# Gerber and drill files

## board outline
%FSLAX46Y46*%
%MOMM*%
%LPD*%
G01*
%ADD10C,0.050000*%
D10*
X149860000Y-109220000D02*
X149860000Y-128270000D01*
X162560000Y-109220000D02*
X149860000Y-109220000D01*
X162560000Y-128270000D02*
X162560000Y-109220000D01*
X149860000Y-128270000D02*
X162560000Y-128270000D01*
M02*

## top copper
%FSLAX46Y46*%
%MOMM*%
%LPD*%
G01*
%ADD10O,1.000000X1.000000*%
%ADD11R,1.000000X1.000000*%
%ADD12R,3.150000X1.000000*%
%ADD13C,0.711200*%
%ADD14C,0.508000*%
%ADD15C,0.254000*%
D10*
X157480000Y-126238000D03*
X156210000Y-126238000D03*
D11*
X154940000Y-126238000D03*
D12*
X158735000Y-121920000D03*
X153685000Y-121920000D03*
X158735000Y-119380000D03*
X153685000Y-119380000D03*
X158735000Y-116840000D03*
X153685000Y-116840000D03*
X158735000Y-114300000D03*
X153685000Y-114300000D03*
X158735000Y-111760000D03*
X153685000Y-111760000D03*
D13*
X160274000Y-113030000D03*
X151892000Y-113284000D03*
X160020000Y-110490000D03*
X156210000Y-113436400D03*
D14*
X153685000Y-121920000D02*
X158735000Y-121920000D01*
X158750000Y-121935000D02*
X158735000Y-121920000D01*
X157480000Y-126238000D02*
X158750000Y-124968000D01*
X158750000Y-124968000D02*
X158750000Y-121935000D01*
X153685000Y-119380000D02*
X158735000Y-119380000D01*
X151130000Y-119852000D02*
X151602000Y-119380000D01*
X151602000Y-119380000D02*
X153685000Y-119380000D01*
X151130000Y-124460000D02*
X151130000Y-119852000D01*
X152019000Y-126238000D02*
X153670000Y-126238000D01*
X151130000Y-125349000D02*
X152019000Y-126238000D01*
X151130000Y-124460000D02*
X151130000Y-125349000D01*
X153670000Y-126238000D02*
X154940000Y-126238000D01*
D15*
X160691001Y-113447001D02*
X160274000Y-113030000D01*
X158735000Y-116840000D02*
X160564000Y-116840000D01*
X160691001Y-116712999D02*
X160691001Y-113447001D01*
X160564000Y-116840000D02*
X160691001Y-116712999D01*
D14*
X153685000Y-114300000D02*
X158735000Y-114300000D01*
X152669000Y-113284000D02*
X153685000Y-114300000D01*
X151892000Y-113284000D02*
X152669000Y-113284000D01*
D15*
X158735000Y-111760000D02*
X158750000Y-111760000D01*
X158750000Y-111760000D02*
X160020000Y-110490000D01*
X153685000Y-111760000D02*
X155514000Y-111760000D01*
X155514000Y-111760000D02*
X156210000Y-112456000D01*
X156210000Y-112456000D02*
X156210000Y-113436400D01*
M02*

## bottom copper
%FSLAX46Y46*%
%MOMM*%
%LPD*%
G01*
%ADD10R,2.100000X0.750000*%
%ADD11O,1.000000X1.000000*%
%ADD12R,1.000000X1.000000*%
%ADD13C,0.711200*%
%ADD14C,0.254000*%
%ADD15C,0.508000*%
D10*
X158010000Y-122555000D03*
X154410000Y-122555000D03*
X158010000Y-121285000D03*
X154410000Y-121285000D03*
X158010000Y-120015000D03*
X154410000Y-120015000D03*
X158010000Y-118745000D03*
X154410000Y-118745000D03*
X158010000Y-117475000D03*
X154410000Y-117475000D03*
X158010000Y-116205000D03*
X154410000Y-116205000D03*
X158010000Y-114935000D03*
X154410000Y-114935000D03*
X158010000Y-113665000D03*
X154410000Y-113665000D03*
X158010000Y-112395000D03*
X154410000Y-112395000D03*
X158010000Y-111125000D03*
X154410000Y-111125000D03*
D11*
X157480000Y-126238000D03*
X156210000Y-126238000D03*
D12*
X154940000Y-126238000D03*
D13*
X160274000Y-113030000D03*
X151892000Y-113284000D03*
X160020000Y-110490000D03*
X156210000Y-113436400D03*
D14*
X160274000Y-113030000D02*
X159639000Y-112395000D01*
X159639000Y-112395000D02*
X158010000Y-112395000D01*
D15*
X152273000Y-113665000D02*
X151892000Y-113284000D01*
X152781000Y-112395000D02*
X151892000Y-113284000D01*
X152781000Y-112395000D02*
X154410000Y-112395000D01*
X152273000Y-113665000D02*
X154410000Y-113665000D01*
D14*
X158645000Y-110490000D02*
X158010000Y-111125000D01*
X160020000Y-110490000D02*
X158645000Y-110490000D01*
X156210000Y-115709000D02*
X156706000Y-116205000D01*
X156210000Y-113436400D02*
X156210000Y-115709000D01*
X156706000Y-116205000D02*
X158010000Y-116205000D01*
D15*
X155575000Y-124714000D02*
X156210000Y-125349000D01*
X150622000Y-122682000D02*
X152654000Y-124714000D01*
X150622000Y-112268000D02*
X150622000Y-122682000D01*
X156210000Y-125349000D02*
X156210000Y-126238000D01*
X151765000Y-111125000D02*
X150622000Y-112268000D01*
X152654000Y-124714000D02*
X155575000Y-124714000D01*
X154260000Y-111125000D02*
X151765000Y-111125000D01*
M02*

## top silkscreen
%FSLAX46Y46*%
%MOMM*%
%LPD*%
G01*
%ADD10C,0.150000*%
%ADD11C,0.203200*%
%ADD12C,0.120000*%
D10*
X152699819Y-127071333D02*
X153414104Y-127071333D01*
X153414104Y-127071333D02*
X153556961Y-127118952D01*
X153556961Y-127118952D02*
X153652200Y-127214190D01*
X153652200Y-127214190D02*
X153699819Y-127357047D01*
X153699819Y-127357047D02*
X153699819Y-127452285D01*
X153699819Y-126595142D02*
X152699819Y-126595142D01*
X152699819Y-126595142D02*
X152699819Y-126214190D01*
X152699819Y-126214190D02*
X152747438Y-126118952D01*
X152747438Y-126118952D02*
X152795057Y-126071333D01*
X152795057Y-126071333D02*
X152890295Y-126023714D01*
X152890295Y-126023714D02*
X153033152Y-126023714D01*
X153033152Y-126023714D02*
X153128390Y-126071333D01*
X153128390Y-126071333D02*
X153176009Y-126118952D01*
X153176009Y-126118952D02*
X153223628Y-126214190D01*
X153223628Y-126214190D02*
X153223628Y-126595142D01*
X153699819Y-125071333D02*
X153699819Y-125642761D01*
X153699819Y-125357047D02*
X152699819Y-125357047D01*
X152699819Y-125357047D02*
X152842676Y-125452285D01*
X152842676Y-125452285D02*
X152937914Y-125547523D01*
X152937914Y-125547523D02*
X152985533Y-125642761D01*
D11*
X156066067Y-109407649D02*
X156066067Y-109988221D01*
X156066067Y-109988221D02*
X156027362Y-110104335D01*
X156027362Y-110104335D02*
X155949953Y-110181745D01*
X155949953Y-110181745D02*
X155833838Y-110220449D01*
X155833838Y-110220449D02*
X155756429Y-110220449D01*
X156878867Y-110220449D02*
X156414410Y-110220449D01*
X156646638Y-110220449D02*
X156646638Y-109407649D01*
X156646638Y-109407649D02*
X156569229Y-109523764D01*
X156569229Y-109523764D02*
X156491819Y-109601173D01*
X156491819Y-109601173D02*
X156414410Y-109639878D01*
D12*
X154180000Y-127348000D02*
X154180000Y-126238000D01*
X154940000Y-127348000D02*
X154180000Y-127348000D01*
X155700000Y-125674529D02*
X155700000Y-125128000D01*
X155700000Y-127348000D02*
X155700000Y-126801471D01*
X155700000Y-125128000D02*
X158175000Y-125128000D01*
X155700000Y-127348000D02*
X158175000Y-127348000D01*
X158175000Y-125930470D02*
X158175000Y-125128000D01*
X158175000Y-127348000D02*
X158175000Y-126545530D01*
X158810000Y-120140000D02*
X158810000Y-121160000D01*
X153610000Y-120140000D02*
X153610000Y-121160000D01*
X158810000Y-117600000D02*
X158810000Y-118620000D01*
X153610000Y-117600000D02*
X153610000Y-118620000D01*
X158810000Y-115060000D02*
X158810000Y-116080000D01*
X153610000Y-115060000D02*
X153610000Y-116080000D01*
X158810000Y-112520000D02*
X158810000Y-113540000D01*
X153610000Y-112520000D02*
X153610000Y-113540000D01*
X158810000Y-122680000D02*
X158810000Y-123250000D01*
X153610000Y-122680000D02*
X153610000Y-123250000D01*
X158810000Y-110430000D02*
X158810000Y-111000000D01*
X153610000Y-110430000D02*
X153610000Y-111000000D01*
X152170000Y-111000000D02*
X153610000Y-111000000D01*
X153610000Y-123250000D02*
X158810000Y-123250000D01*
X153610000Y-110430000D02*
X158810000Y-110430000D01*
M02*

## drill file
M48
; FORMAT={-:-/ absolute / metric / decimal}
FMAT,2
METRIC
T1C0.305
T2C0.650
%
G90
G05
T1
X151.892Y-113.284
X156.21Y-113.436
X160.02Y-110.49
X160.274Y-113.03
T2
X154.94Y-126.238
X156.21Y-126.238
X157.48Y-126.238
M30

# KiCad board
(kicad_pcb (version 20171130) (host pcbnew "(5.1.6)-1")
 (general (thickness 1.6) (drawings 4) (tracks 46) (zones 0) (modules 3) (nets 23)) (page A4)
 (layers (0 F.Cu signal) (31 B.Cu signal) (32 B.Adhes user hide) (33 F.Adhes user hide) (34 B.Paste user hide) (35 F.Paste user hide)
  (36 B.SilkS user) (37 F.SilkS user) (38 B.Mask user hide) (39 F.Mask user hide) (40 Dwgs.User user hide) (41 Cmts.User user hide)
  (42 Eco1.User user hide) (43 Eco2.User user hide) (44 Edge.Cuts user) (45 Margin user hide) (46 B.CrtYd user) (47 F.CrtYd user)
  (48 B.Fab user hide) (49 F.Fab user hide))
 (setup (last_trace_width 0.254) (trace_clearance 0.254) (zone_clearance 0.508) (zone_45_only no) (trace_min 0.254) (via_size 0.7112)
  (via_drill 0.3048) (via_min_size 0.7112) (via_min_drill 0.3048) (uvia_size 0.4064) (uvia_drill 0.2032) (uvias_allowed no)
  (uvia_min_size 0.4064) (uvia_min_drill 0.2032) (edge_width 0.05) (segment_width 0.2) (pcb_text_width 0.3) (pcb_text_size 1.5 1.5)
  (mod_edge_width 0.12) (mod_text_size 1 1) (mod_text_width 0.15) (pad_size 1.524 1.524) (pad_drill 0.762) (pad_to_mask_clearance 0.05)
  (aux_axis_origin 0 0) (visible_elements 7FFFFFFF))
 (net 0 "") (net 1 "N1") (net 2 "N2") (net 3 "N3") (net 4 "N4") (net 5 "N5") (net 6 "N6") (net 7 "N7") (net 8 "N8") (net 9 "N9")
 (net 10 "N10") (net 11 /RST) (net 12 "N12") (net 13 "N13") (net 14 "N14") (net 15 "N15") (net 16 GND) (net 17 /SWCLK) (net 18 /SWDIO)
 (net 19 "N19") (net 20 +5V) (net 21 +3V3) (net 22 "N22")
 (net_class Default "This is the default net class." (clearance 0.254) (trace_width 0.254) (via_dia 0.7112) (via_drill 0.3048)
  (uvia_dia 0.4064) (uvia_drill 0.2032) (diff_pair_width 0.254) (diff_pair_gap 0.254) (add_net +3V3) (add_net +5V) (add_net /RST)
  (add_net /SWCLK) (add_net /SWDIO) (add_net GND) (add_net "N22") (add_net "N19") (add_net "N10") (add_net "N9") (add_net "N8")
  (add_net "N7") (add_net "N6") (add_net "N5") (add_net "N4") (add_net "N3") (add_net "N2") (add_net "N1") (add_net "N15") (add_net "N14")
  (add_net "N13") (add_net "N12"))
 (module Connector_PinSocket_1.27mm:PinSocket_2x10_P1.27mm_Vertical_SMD (layer B.Cu) (at 156.21 116.84 180)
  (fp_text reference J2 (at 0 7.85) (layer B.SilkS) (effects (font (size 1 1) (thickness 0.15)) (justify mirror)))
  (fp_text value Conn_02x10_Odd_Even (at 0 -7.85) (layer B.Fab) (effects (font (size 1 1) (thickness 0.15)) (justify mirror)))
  (pad 20 smd rect (at -1.8 -5.715 180) (size 2.1 0.75) (layers B.Cu B.Paste B.Mask) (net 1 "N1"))
  (pad 19 smd rect (at 1.8 -5.715 180) (size 2.1 0.75) (layers B.Cu B.Paste B.Mask) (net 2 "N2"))
  (pad 18 smd rect (at -1.8 -4.445 180) (size 2.1 0.75) (layers B.Cu B.Paste B.Mask) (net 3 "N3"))
  (pad 17 smd rect (at 1.8 -4.445 180) (size 2.1 0.75) (layers B.Cu B.Paste B.Mask) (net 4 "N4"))
  (pad 16 smd rect (at -1.8 -3.175 180) (size 2.1 0.75) (layers B.Cu B.Paste B.Mask) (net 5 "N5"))
  (pad 15 smd rect (at 1.8 -3.175 180) (size 2.1 0.75) (layers B.Cu B.Paste B.Mask) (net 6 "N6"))
  (pad 14 smd rect (at -1.8 -1.905 180) (size 2.1 0.75) (layers B.Cu B.Paste B.Mask) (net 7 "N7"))
  (pad 13 smd rect (at 1.8 -1.905 180) (size 2.1 0.75) (layers B.Cu B.Paste B.Mask) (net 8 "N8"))
  (pad 12 smd rect (at -1.8 -0.635 180) (size 2.1 0.75) (layers B.Cu B.Paste B.Mask) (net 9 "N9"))
  (pad 11 smd rect (at 1.8 -0.635 180) (size 2.1 0.75) (layers B.Cu B.Paste B.Mask) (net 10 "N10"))
  (pad 10 smd rect (at -1.8 0.635 180) (size 2.1 0.75) (layers B.Cu B.Paste B.Mask) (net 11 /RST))
  (pad 9 smd rect (at 1.8 0.635 180) (size 2.1 0.75) (layers B.Cu B.Paste B.Mask) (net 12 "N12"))
  (pad 8 smd rect (at -1.8 1.905 180) (size 2.1 0.75) (layers B.Cu B.Paste B.Mask) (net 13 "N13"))
  (pad 7 smd rect (at 1.8 1.905 180) (size 2.1 0.75) (layers B.Cu B.Paste B.Mask) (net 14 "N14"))
  (pad 6 smd rect (at -1.8 3.175 180) (size 2.1 0.75) (layers B.Cu B.Paste B.Mask) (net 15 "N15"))
  (pad 5 smd rect (at 1.8 3.175 180) (size 2.1 0.75) (layers B.Cu B.Paste B.Mask) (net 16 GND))
  (pad 4 smd rect (at -1.8 4.445 180) (size 2.1 0.75) (layers B.Cu B.Paste B.Mask) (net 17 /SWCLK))
  (pad 3 smd rect (at 1.8 4.445 180) (size 2.1 0.75) (layers B.Cu B.Paste B.Mask) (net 16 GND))
  (pad 2 smd rect (at -1.8 5.715 180) (size 2.1 0.75) (layers B.Cu B.Paste B.Mask) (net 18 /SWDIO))
  (pad 1 smd rect (at 1.8 5.715 180) (size 2.1 0.75) (layers B.Cu B.Paste B.Mask) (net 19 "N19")))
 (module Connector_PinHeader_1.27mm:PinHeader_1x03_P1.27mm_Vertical (layer F.Cu) (at 154.94 126.238 90)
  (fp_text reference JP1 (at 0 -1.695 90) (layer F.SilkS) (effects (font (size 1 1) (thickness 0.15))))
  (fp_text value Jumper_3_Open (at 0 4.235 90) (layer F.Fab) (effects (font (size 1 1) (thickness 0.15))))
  (fp_line (start -1.11 -0.76) (end 0 -0.76) (layer F.SilkS) (width 0.12))
  (fp_line (start -1.11 0) (end -1.11 -0.76) (layer F.SilkS) (width 0.12))
  (fp_line (start 0.563471 0.76) (end 1.11 0.76) (layer F.SilkS) (width 0.12))
  (fp_line (start -1.11 0.76) (end -0.563471 0.76) (layer F.SilkS) (width 0.12))
  (fp_line (start 1.11 0.76) (end 1.11 3.235) (layer F.SilkS) (width 0.12))
  (fp_line (start -1.11 0.76) (end -1.11 3.235) (layer F.SilkS) (width 0.12))
  (fp_line (start 0.30753 3.235) (end 1.11 3.235) (layer F.SilkS) (width 0.12))
  (fp_line (start -1.11 3.235) (end -0.30753 3.235) (layer F.SilkS) (width 0.12))
  (pad 3 thru_hole oval (at 0 2.54 90) (size 1 1) (drill 0.65) (layers *.Cu *.Mask) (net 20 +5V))
  (pad 2 thru_hole oval (at 0 1.27 90) (size 1 1) (drill 0.65) (layers *.Cu *.Mask) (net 19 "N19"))
  (pad 1 thru_hole rect (at 0 0 90) (size 1 1) (drill 0.65) (layers *.Cu *.Mask) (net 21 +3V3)))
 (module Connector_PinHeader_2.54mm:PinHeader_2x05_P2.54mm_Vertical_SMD (layer F.Cu) (at 156.21 116.84)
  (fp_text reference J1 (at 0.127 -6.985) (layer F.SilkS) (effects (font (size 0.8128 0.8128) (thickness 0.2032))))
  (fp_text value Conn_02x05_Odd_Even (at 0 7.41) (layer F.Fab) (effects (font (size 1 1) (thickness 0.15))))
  (fp_line (start 2.6 3.3) (end 2.6 4.32) (layer F.SilkS) (width 0.12))
  (fp_line (start -2.6 3.3) (end -2.6 4.32) (layer F.SilkS) (width 0.12))
  (fp_line (start 2.6 0.76) (end 2.6 1.78) (layer F.SilkS) (width 0.12))
  (fp_line (start -2.6 0.76) (end -2.6 1.78) (layer F.SilkS) (width 0.12))
  (fp_line (start 2.6 -1.78) (end 2.6 -0.76) (layer F.SilkS) (width 0.12))
  (fp_line (start -2.6 -1.78) (end -2.6 -0.76) (layer F.SilkS) (width 0.12))
  (fp_line (start 2.6 -4.32) (end 2.6 -3.3) (layer F.SilkS) (width 0.12))
  (fp_line (start -2.6 -4.32) (end -2.6 -3.3) (layer F.SilkS) (width 0.12))
  (fp_line (start 2.6 5.84) (end 2.6 6.41) (layer F.SilkS) (width 0.12))
  (fp_line (start -2.6 5.84) (end -2.6 6.41) (layer F.SilkS) (width 0.12))
  (fp_line (start 2.6 -6.41) (end 2.6 -5.84) (layer F.SilkS) (width 0.12))
  (fp_line (start -2.6 -6.41) (end -2.6 -5.84) (layer F.SilkS) (width 0.12))
  (fp_line (start -4.04 -5.84) (end -2.6 -5.84) (layer F.SilkS) (width 0.12))
  (fp_line (start -2.6 6.41) (end 2.6 6.41) (layer F.SilkS) (width 0.12))
  (fp_line (start -2.6 -6.41) (end 2.6 -6.41) (layer F.SilkS) (width 0.12))
  (pad 10 smd rect (at 2.525 5.08) (size 3.15 1) (layers F.Cu F.Paste F.Mask) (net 20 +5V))
  (pad 9 smd rect (at -2.525 5.08) (size 3.15 1) (layers F.Cu F.Paste F.Mask) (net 20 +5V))
  (pad 8 smd rect (at 2.525 2.54) (size 3.15 1) (layers F.Cu F.Paste F.Mask) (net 21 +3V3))
  (pad 7 smd rect (at -2.525 2.54) (size 3.15 1) (layers F.Cu F.Paste F.Mask) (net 21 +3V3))
  (pad 6 smd rect (at 2.525 0) (size 3.15 1) (layers F.Cu F.Paste F.Mask) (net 17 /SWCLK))
  (pad 5 smd rect (at -2.525 0) (size 3.15 1) (layers F.Cu F.Paste F.Mask) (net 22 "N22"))
  (pad 4 smd rect (at 2.525 -2.54) (size 3.15 1) (layers F.Cu F.Paste F.Mask) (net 16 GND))
  (pad 3 smd rect (at -2.525 -2.54) (size 3.15 1) (layers F.Cu F.Paste F.Mask) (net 16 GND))
  (pad 2 smd rect (at 2.525 -5.08) (size 3.15 1) (layers F.Cu F.Paste F.Mask) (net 18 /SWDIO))
  (pad 1 smd rect (at -2.525 -5.08) (size 3.15 1) (layers F.Cu F.Paste F.Mask) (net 11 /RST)))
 (gr_line (start 149.86 109.22) (end 149.86 128.27) (layer Edge.Cuts) (width 0.05))
 (gr_line (start 162.56 109.22) (end 149.86 109.22) (layer Edge.Cuts) (width 0.05))
 (gr_line (start 162.56 128.27) (end 162.56 109.22) (layer Edge.Cuts) (width 0.05))
 (gr_line (start 149.86 128.27) (end 162.56 128.27) (layer Edge.Cuts) (width 0.05))
 (segment (start 153.685 121.92) (end 158.735 121.92) (width 0.508) (layer F.Cu) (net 20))
 (segment (start 158.75 121.935) (end 158.735 121.92) (width 0.508) (layer F.Cu) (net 20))
 (segment (start 157.48 126.238) (end 158.75 124.968) (width 0.508) (layer F.Cu) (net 20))
 (segment (start 158.75 124.968) (end 158.75 121.935) (width 0.508) (layer F.Cu) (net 20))
 (segment (start 153.685 119.38) (end 158.735 119.38) (width 0.508) (layer F.Cu) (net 21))
 (segment (start 151.13 119.852) (end 151.602 119.38) (width 0.508) (layer F.Cu) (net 21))
 (segment (start 151.602 119.38) (end 153.685 119.38) (width 0.508) (layer F.Cu) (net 21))
 (segment (start 151.13 124.46) (end 151.13 119.852) (width 0.508) (layer F.Cu) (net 21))
 (segment (start 152.019 126.238) (end 153.67 126.238) (width 0.508) (layer F.Cu) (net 21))
 (segment (start 151.13 125.349) (end 152.019 126.238) (width 0.508) (layer F.Cu) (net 21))
 (segment (start 151.13 124.46) (end 151.13 125.349) (width 0.508) (layer F.Cu) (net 21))
 (segment (start 153.67 126.238) (end 154.94 126.238) (width 0.508) (layer F.Cu) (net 21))
 (segment (start 160.691001 113.447001) (end 160.274 113.03) (width 0.254) (layer F.Cu) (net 17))
 (via (at 160.274 113.03) (size 0.7112) (drill 0.3048) (layers F.Cu B.Cu) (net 17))
 (segment (start 158.735 116.84) (end 160.564 116.84) (width 0.254) (layer F.Cu) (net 17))
 (segment (start 160.691001 116.712999) (end 160.691001 113.447001) (width 0.254) (layer F.Cu) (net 17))
 (segment (start 160.564 116.84) (end 160.691001 116.712999) (width 0.254) (layer F.Cu) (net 17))
 (segment (start 160.274 113.03) (end 159.639 112.395) (width 0.254) (layer B.Cu) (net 17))
 (segment (start 159.639 112.395) (end 158.01 112.395) (width 0.254) (layer B.Cu) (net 17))
 (segment (start 153.685 114.3) (end 158.735 114.3) (width 0.508) (layer F.Cu) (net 16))
 (via (at 151.892 113.284) (size 0.7112) (drill 0.3048) (layers F.Cu B.Cu) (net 16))
 (segment (start 152.273 113.665) (end 151.892 113.284) (width 0.508) (layer B.Cu) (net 16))
 (segment (start 152.669 113.284) (end 153.685 114.3) (width 0.508) (layer F.Cu) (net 16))
 (segment (start 151.892 113.284) (end 152.669 113.284) (width 0.508) (layer F.Cu) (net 16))
 (segment (start 152.781 112.395) (end 151.892 113.284) (width 0.508) (layer B.Cu) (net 16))
 (segment (start 152.781 112.395) (end 154.41 112.395) (width 0.508) (layer B.Cu) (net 16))
 (segment (start 152.273 113.665) (end 154.41 113.665) (width 0.508) (layer B.Cu) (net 16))
 (via (at 160.02 110.49) (size 0.7112) (drill 0.3048) (layers F.Cu B.Cu) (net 18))
 (segment (start 158.735 111.76) (end 158.75 111.76) (width 0.254) (layer F.Cu) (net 18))
 (segment (start 158.75 111.76) (end 160.02 110.49) (width 0.254) (layer F.Cu) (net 18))
 (segment (start 158.645 110.49) (end 158.01 111.125) (width 0.254) (layer B.Cu) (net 18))
 (segment (start 160.02 110.49) (end 158.645 110.49) (width 0.254) (layer B.Cu) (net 18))
 (segment (start 153.685 111.76) (end 155.514 111.76) (width 0.254) (layer F.Cu) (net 11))
 (segment (start 155.514 111.76) (end 156.21 112.456) (width 0.254) (layer F.Cu) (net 11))
 (via (at 156.21 113.4364) (size 0.7112) (drill 0.3048) (layers F.Cu B.Cu) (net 11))
 (segment (start 156.21 112.456) (end 156.21 113.4364) (width 0.254) (layer F.Cu) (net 11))
 (segment (start 156.21 115.709) (end 156.706 116.205) (width 0.254) (layer B.Cu) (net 11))
 (segment (start 156.21 113.4364) (end 156.21 115.709) (width 0.254) (layer B.Cu) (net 11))
 (segment (start 156.706 116.205) (end 158.01 116.205) (width 0.254) (layer B.Cu) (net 11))
 (segment (start 155.575 124.714) (end 156.21 125.349) (width 0.508) (layer B.Cu) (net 19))
 (segment (start 150.622 122.682) (end 152.654 124.714) (width 0.508) (layer B.Cu) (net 19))
 (segment (start 150.622 112.268) (end 150.622 122.682) (width 0.508) (layer B.Cu) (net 19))
 (segment (start 156.21 125.349) (end 156.21 126.238) (width 0.508) (layer B.Cu) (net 19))
 (segment (start 151.765 111.125) (end 150.622 112.268) (width 0.508) (layer B.Cu) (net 19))
 (segment (start 152.654 124.714) (end 155.575 124.714) (width 0.508) (layer B.Cu) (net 19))
 (segment (start 154.26 111.125) (end 151.765 111.125) (width 0.508) (layer B.Cu) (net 19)))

